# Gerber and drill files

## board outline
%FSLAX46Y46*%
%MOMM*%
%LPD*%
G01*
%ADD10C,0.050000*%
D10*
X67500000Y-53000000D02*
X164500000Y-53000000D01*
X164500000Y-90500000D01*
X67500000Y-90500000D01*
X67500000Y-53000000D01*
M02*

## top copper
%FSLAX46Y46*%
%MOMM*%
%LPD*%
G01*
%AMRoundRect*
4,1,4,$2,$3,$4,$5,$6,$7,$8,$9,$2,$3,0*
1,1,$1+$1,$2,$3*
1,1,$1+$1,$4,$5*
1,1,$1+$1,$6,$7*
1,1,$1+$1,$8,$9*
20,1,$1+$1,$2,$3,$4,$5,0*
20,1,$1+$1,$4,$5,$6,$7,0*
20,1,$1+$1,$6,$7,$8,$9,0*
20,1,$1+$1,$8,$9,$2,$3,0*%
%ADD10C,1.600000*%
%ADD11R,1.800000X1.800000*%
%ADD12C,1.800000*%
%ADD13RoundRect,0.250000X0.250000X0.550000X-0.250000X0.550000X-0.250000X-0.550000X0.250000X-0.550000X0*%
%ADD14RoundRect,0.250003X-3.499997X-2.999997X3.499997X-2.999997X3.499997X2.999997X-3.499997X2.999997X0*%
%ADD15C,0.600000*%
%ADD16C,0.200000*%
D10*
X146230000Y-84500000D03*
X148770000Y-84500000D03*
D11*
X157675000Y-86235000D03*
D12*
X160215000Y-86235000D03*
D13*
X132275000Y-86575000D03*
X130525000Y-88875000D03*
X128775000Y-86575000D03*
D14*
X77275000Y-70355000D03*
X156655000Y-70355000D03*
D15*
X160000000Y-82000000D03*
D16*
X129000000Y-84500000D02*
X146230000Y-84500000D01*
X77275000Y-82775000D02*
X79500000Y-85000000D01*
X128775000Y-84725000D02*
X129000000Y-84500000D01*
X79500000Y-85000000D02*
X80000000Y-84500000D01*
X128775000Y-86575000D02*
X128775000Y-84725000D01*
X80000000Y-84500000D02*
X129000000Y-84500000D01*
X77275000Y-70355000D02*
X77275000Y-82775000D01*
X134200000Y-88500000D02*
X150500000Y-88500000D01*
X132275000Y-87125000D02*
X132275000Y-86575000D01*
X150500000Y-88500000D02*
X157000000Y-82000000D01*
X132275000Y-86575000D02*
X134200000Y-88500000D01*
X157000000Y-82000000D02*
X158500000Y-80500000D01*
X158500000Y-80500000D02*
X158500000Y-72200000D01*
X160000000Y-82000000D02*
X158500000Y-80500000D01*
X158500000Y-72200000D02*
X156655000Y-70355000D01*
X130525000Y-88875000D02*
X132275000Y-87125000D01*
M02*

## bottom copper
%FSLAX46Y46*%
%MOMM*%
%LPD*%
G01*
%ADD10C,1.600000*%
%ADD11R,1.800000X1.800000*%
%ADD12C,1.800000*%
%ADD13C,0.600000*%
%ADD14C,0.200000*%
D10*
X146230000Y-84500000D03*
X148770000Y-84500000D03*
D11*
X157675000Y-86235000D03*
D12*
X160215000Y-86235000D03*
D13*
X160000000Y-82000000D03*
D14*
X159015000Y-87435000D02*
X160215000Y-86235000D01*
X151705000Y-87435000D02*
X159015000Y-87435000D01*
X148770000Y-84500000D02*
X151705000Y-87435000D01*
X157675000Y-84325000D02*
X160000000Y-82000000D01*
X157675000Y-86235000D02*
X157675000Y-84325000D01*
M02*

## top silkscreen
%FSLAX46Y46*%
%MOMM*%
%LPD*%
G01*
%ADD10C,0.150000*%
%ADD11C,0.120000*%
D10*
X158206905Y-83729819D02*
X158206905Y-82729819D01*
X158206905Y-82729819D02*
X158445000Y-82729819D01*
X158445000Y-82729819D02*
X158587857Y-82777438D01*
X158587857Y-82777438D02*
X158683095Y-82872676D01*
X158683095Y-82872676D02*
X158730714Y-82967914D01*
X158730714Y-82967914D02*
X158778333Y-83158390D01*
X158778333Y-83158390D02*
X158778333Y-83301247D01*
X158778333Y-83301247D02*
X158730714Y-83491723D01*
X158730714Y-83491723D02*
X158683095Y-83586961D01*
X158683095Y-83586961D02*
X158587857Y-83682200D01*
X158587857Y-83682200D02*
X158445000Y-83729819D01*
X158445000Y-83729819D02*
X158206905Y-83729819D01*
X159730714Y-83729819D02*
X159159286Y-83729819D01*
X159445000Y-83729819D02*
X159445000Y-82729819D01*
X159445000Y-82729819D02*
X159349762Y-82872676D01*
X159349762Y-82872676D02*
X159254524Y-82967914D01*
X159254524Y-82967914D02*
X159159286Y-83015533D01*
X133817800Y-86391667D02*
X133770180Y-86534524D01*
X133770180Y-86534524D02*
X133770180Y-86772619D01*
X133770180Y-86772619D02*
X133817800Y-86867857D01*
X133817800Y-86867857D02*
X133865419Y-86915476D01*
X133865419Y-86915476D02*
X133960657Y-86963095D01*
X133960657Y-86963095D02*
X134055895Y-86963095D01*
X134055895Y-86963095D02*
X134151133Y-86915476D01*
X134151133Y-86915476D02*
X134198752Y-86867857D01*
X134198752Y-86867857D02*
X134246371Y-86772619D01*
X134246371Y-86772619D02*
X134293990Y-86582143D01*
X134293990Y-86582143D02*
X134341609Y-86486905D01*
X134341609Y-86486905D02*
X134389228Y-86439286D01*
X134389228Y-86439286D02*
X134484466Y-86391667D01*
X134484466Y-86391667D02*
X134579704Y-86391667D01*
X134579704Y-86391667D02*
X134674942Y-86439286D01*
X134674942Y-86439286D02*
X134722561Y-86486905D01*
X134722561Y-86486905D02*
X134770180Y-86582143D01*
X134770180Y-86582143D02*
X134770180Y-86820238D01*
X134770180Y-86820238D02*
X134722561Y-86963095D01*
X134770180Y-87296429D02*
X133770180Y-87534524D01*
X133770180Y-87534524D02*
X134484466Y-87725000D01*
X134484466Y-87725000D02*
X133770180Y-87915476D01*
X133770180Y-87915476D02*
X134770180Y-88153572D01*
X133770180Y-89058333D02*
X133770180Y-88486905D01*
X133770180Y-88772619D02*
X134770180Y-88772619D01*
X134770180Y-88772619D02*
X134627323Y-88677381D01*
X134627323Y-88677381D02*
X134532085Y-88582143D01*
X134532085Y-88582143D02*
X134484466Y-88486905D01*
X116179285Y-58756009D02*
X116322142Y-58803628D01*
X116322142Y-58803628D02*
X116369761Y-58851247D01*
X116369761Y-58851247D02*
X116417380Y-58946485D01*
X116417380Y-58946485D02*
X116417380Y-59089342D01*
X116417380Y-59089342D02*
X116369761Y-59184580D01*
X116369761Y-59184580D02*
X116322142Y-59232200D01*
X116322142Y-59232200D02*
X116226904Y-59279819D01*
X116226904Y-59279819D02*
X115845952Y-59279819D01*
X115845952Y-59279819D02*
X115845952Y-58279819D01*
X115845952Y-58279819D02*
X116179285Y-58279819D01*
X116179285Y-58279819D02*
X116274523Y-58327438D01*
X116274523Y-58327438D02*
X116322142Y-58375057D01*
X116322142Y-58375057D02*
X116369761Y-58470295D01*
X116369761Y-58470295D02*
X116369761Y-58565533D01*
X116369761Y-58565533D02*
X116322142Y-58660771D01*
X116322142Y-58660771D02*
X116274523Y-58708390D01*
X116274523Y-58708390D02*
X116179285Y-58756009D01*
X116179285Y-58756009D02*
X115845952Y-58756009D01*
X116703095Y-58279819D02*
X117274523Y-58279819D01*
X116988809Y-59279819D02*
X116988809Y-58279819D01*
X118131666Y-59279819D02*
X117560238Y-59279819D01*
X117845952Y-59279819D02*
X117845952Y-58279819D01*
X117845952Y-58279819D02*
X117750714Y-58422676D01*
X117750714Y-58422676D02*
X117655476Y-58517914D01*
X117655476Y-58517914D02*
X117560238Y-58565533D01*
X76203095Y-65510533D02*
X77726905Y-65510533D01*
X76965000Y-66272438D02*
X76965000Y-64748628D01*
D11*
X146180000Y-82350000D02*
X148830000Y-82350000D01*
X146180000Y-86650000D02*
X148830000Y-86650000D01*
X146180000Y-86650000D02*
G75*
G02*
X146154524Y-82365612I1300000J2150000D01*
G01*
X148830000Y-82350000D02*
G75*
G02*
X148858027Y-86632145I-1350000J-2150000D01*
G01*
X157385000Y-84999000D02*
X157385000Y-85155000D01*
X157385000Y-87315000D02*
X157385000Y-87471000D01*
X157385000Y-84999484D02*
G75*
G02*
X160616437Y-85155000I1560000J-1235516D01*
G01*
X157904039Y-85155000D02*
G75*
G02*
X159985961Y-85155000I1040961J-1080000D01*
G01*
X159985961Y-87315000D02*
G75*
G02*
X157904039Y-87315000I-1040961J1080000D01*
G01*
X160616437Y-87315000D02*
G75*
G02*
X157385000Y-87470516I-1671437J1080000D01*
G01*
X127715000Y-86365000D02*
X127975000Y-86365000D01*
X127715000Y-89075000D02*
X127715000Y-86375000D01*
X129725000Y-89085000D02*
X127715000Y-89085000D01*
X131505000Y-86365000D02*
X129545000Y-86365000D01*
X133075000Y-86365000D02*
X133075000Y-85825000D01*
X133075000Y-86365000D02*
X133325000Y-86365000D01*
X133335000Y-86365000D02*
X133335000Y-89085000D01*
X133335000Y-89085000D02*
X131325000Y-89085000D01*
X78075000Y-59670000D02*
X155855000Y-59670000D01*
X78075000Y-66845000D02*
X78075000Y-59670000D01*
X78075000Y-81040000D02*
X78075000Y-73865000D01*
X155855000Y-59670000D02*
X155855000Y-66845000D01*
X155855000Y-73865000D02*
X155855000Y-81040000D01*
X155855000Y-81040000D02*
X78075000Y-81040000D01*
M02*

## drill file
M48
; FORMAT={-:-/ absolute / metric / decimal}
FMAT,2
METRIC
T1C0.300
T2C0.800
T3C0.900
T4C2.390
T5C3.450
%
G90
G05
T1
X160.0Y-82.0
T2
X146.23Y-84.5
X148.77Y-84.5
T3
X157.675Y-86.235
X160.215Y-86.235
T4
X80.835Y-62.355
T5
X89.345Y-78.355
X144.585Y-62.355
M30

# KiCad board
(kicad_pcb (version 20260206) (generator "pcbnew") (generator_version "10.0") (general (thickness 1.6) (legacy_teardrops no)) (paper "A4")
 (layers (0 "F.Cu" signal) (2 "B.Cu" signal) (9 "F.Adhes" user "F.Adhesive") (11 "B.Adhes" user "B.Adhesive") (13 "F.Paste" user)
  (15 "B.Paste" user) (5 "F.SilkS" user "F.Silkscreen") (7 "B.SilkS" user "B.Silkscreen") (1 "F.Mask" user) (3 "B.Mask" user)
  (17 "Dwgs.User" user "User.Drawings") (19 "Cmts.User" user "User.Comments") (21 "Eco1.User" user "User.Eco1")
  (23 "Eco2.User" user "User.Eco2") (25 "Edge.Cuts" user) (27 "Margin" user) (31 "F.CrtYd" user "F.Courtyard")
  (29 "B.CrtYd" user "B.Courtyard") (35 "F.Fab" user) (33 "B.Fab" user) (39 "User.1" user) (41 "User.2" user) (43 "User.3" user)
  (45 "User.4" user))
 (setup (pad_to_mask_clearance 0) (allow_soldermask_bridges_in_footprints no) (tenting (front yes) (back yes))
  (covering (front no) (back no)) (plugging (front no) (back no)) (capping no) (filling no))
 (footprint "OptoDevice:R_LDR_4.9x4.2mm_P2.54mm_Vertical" (layer "F.Cu") (at 146.23 84.5)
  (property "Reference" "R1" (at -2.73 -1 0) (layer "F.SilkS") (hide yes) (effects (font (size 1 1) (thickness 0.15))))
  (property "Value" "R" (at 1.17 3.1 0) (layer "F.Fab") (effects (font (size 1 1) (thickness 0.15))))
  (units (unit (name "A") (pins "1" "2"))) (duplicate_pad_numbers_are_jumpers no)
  (fp_line (start -0.05 -2.15) (end 2.6 -2.15) (stroke (width 0.12) (type solid)) (layer "F.SilkS"))
  (fp_line (start -0.05 2.15) (end 2.6 2.15) (stroke (width 0.12) (type solid)) (layer "F.SilkS"))
  (fp_arc (start -0.05 2.15) (mid -1.262424 0.01494) (end -0.075476 -2.134388) (stroke (width 0.12) (type solid)) (layer "F.SilkS"))
  (fp_arc (start 2.6 -2.15) (mid 3.788646 -0.016616) (end 2.628027 2.132145) (stroke (width 0.12) (type solid)) (layer "F.SilkS"))
  (pad "1" thru_hole circle (at 0 0) (size 1.6 1.6) (drill 0.8) (layers "*.Cu" "*.Mask") (remove_unused_layers no) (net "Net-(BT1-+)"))
  (pad "2" thru_hole circle (at 2.54 0) (size 1.6 1.6) (drill 0.8) (layers "*.Cu" "*.Mask") (remove_unused_layers no) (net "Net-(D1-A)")))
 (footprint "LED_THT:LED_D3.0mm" (layer "F.Cu") (at 157.675 86.235)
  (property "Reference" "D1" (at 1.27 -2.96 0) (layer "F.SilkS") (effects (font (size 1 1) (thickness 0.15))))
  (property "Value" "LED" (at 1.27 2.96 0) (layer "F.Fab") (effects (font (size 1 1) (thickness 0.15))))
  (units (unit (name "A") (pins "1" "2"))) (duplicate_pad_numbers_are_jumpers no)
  (fp_line (start -0.29 -1.236) (end -0.29 -1.08) (stroke (width 0.12) (type solid)) (layer "F.SilkS"))
  (fp_line (start -0.29 1.08) (end -0.29 1.236) (stroke (width 0.12) (type solid)) (layer "F.SilkS"))
  (fp_arc (start -0.29 -1.235516) (mid 1.36566 -1.987699) (end 2.941437 -1.08) (stroke (width 0.12) (type solid)) (layer "F.SilkS"))
  (fp_arc (start 0.229039 -1.08) (mid 1.27 -1.5) (end 2.310961 -1.08) (stroke (width 0.12) (type solid)) (layer "F.SilkS"))
  (fp_arc (start 2.310961 1.08) (mid 1.27 1.5) (end 0.229039 1.08) (stroke (width 0.12) (type solid)) (layer "F.SilkS"))
  (fp_arc (start 2.941437 1.08) (mid 1.36566 1.987699) (end -0.29 1.235516) (stroke (width 0.12) (type solid)) (layer "F.SilkS"))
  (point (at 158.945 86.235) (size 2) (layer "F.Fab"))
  (pad "1" thru_hole rect (at 0 0) (size 1.8 1.8) (drill 0.9) (layers "*.Cu" "*.Mask") (remove_unused_layers no) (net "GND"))
  (pad "2" thru_hole circle (at 2.54 0) (size 1.8 1.8) (drill 0.9) (layers "*.Cu" "*.Mask") (remove_unused_layers no) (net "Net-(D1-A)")))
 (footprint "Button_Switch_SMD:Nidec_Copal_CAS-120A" (layer "F.Cu") (at 130.525 87.725 -90)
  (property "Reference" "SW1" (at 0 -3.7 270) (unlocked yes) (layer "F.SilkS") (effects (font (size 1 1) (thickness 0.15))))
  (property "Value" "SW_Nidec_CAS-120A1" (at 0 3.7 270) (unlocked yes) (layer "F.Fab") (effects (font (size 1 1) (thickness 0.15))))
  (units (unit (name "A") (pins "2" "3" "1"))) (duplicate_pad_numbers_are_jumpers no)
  (fp_line (start -1.36 2.81) (end -1.36 2.55) (stroke (width 0.12) (type solid)) (layer "F.SilkS"))
  (fp_line (start 1.35 2.81) (end -1.35 2.81) (stroke (width 0.12) (type solid)) (layer "F.SilkS"))
  (fp_line (start 1.36 0.8) (end 1.36 2.81) (stroke (width 0.12) (type solid)) (layer "F.SilkS"))
  (fp_line (start -1.36 -0.98) (end -1.36 0.98) (stroke (width 0.12) (type solid)) (layer "F.SilkS"))
  (fp_line (start -1.36 -2.55) (end -1.9 -2.55) (stroke (width 0.12) (type default)) (layer "F.SilkS"))
  (fp_line (start -1.36 -2.55) (end -1.36 -2.8) (stroke (width 0.12) (type solid)) (layer "F.SilkS"))
  (fp_line (start -1.36 -2.81) (end 1.36 -2.81) (stroke (width 0.12) (type solid)) (layer "F.SilkS"))
  (fp_line (start 1.36 -2.81) (end 1.36 -0.8) (stroke (width 0.12) (type solid)) (layer "F.SilkS"))
  (pad "1" smd roundrect (at -1.15 -1.75 180) (size 1 1.6) (layers "F.Cu" "F.Mask" "F.Paste") (roundrect_rratio 0.25) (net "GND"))
  (pad "2" smd roundrect (at 1.15 0 180) (size 1 1.6) (layers "F.Cu" "F.Mask" "F.Paste") (roundrect_rratio 0.25) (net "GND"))
  (pad "3" smd roundrect (at -1.15 1.75 180) (size 1 1.6) (layers "F.Cu" "F.Mask" "F.Paste") (roundrect_rratio 0.25) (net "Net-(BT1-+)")))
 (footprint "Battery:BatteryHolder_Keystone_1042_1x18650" (layer "F.Cu") (at 116.965 70.355)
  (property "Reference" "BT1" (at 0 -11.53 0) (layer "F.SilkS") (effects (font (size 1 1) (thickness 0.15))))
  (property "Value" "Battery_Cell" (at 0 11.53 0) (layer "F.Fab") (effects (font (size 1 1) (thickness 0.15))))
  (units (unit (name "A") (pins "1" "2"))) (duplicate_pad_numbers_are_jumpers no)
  (fp_line (start -38.89 -10.685) (end 38.89 -10.685) (stroke (width 0.12) (type solid)) (layer "F.SilkS"))
  (fp_line (start -38.89 -3.51) (end -38.89 -10.685) (stroke (width 0.12) (type solid)) (layer "F.SilkS"))
  (fp_line (start -38.89 10.685) (end -38.89 3.51) (stroke (width 0.12) (type solid)) (layer "F.SilkS"))
  (fp_line (start 38.89 -10.685) (end 38.89 -3.51) (stroke (width 0.12) (type solid)) (layer "F.SilkS"))
  (fp_line (start 38.89 3.51) (end 38.89 10.685) (stroke (width 0.12) (type solid)) (layer "F.SilkS"))
  (fp_line (start 38.89 10.685) (end -38.89 10.685) (stroke (width 0.12) (type solid)) (layer "F.SilkS"))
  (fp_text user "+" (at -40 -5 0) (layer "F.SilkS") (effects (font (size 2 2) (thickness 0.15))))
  (pad "" np_thru_hole circle (at -36.13 -8) (size 2.39 2.39) (drill 2.39) (layers "*.Cu" "*.Mask"))
  (pad "" np_thru_hole circle (at -27.62 8) (size 3.45 3.45) (drill 3.45) (layers "*.Cu" "*.Mask"))
  (pad "" np_thru_hole circle (at 27.62 -8) (size 3.45 3.45) (drill 3.45) (layers "*.Cu" "*.Mask"))
  (pad "1" smd roundrect (at -39.69 0) (size 7.5 6.5) (layers "F.Cu" "F.Mask" "F.Paste") (roundrect_rratio 0.038462) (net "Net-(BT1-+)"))
  (pad "2" smd roundrect (at 39.69 0) (size 7.5 6.5) (layers "F.Cu" "F.Mask" "F.Paste") (roundrect_rratio 0.038462) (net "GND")))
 (gr_rect (start 67.5 53) (end 164.5 90.5) (stroke (width 0.05) (type default)) (fill no) (layer "Edge.Cuts"))
 (segment (start 129 84.5) (end 146.23 84.5) (width 0.2) (layer "F.Cu") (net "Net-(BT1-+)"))
 (segment (start 77.275 82.775) (end 79.5 85) (width 0.2) (layer "F.Cu") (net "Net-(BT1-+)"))
 (segment (start 128.775 84.725) (end 129 84.5) (width 0.2) (layer "F.Cu") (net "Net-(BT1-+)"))
 (segment (start 79.5 85) (end 80 84.5) (width 0.2) (layer "F.Cu") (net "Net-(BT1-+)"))
 (segment (start 128.775 86.575) (end 128.775 84.725) (width 0.2) (layer "F.Cu") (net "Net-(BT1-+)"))
 (segment (start 80 84.5) (end 129 84.5) (width 0.2) (layer "F.Cu") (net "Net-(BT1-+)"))
 (segment (start 77.275 70.355) (end 77.275 82.775) (width 0.2) (layer "F.Cu") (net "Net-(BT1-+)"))
 (segment (start 159.015 87.435) (end 160.215 86.235) (width 0.2) (layer "B.Cu") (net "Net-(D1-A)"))
 (segment (start 151.705 87.435) (end 159.015 87.435) (width 0.2) (layer "B.Cu") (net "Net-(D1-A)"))
 (segment (start 148.77 84.5) (end 151.705 87.435) (width 0.2) (layer "B.Cu") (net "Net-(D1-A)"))
 (segment (start 134.2 88.5) (end 150.5 88.5) (width 0.2) (layer "F.Cu") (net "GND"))
 (segment (start 132.275 87.125) (end 132.275 86.575) (width 0.2) (layer "F.Cu") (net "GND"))
 (segment (start 150.5 88.5) (end 157 82) (width 0.2) (layer "F.Cu") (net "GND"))
 (segment (start 132.275 86.575) (end 134.2 88.5) (width 0.2) (layer "F.Cu") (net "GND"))
 (segment (start 157 82) (end 158.5 80.5) (width 0.2) (layer "F.Cu") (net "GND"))
 (segment (start 158.5 80.5) (end 158.5 72.2) (width 0.2) (layer "F.Cu") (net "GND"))
 (segment (start 160 82) (end 158.5 80.5) (width 0.2) (layer "F.Cu") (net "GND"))
 (segment (start 158.5 72.2) (end 156.655 70.355) (width 0.2) (layer "F.Cu") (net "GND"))
 (segment (start 130.525 88.875) (end 132.275 87.125) (width 0.2) (layer "F.Cu") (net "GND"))
 (via (at 160 82) (size 0.6) (drill 0.3) (layers "F.Cu" "B.Cu") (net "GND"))
 (segment (start 157.675 84.325) (end 160 82) (width 0.2) (layer "B.Cu") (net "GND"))
 (segment (start 157.675 86.235) (end 157.675 84.325) (width 0.2) (layer "B.Cu") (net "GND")))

